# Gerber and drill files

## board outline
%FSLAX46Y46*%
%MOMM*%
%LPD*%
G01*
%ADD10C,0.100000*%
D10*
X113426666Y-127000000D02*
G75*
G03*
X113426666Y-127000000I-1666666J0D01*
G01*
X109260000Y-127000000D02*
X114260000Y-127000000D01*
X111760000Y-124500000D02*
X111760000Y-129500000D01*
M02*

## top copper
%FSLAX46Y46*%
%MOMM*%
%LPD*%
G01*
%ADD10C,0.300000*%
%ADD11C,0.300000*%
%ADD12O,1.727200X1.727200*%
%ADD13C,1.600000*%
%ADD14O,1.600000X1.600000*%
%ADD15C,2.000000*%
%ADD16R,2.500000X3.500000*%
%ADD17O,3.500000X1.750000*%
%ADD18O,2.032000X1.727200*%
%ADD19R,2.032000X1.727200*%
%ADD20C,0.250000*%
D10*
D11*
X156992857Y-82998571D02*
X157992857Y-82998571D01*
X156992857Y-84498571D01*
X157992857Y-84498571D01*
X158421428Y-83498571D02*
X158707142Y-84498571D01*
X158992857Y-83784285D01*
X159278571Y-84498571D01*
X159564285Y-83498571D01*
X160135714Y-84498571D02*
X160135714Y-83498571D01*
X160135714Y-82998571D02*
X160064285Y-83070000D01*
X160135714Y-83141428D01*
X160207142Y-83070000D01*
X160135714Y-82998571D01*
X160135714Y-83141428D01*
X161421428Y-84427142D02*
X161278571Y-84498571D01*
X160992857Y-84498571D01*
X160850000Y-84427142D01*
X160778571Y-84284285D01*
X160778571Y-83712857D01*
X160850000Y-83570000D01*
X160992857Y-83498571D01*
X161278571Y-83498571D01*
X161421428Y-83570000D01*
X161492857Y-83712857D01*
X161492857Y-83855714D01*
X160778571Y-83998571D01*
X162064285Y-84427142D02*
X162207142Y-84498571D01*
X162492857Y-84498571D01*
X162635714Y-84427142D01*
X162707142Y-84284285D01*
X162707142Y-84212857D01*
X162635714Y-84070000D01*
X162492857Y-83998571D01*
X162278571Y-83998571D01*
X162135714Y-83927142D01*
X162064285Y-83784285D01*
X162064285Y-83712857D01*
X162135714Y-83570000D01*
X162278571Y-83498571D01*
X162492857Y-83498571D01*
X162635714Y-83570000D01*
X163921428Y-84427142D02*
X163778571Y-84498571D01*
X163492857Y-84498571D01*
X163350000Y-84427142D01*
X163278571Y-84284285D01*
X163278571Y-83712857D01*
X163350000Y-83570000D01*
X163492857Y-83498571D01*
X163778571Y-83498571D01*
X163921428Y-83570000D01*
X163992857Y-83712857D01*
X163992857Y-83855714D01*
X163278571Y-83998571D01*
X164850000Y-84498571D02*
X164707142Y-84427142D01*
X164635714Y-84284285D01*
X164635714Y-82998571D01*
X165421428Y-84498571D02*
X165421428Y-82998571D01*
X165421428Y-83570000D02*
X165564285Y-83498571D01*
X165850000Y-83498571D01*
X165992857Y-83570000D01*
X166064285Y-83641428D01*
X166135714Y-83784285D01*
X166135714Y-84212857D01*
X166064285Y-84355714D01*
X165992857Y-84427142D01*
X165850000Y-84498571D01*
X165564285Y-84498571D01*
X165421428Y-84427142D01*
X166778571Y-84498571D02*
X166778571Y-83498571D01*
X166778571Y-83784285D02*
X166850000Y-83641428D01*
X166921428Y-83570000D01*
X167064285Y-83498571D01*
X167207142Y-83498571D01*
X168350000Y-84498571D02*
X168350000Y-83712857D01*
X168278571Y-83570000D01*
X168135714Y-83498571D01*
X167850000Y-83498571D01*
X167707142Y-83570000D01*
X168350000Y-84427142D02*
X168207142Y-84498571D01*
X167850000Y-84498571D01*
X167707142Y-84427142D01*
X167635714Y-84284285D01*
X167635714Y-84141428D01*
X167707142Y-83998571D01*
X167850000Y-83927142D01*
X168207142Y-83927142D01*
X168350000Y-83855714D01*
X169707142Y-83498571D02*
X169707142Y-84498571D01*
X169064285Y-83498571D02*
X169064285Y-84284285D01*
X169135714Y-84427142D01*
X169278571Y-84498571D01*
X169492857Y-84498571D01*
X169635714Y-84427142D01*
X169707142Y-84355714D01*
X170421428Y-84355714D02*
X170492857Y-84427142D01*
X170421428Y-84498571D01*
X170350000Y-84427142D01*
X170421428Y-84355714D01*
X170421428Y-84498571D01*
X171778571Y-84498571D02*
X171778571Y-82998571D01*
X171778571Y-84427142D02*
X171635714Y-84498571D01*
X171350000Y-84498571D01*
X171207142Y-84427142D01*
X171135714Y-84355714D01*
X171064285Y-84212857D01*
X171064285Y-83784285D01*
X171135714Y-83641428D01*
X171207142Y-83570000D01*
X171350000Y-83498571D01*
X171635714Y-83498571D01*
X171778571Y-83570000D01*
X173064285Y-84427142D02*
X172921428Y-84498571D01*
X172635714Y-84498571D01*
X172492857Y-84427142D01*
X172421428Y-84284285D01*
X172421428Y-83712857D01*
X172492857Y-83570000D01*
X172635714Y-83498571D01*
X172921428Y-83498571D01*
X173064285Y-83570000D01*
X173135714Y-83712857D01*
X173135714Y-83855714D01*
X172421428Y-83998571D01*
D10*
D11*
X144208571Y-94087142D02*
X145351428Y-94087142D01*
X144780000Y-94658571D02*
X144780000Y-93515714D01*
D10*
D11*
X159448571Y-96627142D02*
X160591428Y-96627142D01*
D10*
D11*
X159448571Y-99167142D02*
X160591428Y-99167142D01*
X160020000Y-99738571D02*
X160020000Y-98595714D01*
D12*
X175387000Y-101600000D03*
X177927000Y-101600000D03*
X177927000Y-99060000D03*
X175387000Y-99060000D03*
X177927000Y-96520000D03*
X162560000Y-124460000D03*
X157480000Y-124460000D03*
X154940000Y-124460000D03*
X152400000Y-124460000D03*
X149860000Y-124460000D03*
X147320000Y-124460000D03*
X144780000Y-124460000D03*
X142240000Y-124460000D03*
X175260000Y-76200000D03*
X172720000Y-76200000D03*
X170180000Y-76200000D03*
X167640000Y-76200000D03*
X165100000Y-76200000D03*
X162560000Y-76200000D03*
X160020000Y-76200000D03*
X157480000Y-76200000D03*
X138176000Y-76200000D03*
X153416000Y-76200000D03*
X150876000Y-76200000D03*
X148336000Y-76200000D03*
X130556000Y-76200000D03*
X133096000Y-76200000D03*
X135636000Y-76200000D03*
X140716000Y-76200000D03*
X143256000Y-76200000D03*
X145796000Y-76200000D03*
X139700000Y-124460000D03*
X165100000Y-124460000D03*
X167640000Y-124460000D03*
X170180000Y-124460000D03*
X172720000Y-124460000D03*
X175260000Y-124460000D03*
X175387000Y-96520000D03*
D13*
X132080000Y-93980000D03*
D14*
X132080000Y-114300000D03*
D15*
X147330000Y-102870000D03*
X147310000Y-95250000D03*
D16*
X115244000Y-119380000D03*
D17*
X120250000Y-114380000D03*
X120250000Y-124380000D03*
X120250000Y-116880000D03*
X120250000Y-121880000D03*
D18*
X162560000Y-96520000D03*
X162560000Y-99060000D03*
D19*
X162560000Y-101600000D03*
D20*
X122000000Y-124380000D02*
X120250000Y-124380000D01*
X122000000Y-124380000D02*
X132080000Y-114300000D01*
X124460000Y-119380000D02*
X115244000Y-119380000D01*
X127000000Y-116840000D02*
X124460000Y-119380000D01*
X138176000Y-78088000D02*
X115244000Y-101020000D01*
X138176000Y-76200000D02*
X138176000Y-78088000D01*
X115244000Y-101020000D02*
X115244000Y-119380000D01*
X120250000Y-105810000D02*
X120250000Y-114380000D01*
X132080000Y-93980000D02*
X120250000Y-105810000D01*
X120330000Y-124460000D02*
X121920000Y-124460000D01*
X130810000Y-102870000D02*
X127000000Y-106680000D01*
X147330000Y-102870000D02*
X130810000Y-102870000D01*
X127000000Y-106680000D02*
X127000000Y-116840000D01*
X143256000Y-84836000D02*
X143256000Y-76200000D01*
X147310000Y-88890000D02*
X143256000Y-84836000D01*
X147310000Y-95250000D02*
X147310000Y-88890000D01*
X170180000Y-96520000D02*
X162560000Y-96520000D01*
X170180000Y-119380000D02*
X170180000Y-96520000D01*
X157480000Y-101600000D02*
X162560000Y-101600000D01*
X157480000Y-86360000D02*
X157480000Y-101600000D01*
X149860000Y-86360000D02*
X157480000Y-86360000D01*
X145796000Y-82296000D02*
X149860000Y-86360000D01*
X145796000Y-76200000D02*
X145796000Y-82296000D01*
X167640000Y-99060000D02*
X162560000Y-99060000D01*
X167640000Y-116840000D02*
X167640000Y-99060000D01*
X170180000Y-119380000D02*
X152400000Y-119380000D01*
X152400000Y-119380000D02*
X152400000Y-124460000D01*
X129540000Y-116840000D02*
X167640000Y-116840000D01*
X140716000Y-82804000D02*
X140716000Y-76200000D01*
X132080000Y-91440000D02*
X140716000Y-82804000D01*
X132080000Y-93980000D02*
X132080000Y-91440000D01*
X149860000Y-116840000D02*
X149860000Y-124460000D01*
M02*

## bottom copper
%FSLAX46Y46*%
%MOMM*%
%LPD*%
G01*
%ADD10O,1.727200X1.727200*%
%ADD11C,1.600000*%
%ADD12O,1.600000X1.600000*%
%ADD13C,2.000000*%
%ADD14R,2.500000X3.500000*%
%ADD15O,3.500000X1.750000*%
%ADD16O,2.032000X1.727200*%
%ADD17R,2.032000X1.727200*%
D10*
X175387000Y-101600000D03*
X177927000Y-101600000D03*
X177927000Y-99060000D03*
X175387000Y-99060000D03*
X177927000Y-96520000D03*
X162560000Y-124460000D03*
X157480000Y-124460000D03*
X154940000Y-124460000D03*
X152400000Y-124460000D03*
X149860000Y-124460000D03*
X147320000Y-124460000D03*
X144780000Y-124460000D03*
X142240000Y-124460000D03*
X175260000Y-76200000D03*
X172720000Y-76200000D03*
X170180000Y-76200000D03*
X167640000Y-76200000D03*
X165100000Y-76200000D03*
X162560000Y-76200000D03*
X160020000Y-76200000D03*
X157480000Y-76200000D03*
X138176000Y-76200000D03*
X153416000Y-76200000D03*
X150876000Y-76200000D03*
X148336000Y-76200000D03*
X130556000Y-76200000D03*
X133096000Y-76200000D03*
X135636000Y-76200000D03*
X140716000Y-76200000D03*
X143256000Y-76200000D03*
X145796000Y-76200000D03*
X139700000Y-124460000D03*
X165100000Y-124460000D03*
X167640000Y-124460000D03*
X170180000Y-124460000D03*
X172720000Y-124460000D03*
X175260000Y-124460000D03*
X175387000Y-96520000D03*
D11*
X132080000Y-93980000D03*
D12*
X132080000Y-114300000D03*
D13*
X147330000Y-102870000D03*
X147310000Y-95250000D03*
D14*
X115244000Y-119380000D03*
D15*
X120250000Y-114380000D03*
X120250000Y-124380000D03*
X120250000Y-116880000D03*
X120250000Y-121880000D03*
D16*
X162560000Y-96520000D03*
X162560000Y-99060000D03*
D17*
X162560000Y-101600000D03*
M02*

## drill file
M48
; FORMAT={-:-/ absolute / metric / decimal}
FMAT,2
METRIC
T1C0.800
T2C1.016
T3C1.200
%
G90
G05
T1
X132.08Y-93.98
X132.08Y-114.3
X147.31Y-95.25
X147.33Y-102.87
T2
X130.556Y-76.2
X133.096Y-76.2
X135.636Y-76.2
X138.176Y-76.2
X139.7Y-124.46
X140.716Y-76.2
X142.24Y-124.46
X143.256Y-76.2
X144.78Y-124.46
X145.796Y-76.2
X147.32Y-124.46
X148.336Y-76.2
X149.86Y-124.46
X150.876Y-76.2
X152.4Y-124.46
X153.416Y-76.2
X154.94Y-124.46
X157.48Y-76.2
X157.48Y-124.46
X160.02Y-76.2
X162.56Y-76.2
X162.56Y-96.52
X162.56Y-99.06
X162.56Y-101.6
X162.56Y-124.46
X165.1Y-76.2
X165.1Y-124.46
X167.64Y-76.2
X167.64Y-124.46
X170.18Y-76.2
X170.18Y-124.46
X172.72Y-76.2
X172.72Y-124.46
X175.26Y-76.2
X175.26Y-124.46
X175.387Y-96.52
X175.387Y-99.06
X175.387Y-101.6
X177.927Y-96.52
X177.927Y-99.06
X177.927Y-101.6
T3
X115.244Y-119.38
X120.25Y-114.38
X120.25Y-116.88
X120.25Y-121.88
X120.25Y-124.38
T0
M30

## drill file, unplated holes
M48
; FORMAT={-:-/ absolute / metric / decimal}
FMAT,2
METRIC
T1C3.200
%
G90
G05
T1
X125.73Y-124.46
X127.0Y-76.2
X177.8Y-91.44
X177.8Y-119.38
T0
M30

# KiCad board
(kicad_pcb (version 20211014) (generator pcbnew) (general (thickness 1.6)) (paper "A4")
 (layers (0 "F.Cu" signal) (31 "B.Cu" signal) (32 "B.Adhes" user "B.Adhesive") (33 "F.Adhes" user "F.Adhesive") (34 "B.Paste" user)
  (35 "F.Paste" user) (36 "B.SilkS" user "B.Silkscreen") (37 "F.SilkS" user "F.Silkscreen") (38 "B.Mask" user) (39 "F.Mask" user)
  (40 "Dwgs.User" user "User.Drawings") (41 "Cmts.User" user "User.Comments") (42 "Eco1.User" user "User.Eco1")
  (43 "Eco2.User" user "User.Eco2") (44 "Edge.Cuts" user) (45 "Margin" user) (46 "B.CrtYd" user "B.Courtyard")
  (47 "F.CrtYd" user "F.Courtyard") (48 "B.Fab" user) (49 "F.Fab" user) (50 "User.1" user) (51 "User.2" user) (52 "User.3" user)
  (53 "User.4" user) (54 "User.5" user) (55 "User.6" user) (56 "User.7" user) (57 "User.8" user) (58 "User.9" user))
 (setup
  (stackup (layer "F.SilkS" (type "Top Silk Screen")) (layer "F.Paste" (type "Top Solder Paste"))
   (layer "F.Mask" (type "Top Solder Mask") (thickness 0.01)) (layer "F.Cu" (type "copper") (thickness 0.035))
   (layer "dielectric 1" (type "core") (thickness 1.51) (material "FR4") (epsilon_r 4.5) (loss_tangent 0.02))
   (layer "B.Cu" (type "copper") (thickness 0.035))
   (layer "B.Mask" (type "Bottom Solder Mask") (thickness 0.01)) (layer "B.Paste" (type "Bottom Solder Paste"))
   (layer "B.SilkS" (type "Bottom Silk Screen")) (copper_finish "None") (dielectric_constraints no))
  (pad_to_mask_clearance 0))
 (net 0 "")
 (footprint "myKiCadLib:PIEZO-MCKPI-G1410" (layer "F.Cu") (at 147.32 99.06 90)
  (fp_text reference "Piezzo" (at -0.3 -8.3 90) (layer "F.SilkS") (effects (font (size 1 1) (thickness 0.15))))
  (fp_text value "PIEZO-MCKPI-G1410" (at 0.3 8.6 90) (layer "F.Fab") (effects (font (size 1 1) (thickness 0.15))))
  (pad "1" thru_hole circle locked (at -3.81 0.01 90) (size 2 2) (drill 0.8) (layers *.Cu *.Mask "F.SilkS"))
  (pad "2" thru_hole circle locked (at 3.81 -0.01 90) (size 2 2) (drill 0.8) (layers *.Cu *.Mask "F.SilkS")))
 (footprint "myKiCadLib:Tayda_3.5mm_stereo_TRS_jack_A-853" (layer "F.Cu") (at 116.84 119.38 90)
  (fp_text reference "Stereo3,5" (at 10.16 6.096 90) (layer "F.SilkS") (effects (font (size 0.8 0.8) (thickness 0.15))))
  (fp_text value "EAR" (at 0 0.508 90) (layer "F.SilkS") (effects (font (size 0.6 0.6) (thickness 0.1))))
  (pad "1" thru_hole rect locked (at 0 -1.596 90) (size 3.5 2.5) (drill 1.2) (layers *.Cu *.Mask "F.SilkS"))
  (pad "2" thru_hole oval locked (at 5 3.41 90) (size 1.75 3.5) (drill 1.2) (layers *.Cu *.Mask "F.SilkS"))
  (pad "3" thru_hole oval locked (at 2.5 3.41 90) (size 1.75 3.5) (drill 1.2) (layers *.Cu *.Mask "F.SilkS"))
  (pad "4" thru_hole oval locked (at -2.5 3.41 90) (size 1.75 3.5) (drill 1.2) (layers *.Cu *.Mask "F.SilkS"))
  (pad "5" thru_hole oval locked (at -5 3.41 90) (size 1.75 3.5) (drill 1.2) (layers *.Cu *.Mask "F.SilkS")))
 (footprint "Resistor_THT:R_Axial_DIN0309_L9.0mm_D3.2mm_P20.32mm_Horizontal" (layer "F.Cu") (at 132.08 93.98 -90)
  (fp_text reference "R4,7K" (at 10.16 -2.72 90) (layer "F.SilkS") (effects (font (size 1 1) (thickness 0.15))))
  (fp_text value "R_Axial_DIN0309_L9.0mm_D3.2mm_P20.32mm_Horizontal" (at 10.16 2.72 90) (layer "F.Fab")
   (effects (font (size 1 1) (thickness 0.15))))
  (pad "1" thru_hole circle (at 0 0 270) (size 1.6 1.6) (drill 0.8) (layers *.Cu *.Mask))
  (pad "2" thru_hole oval (at 20.32 0 270) (size 1.6 1.6) (drill 0.8) (layers *.Cu *.Mask)))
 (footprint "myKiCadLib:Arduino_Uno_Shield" (layer "F.Cu") (at 111.76 127)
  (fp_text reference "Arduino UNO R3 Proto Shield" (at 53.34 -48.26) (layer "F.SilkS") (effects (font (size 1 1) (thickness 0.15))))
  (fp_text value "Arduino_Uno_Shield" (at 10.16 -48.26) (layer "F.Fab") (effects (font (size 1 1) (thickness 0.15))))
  (pad "" np_thru_hole circle locked (at 15.24 -50.8) (size 3.2 3.2) (drill 3.2) (layers *.Cu *.Mask))
  (pad "" np_thru_hole circle locked (at 66.04 -7.62) (size 3.2 3.2) (drill 3.2) (layers *.Cu *.Mask))
  (pad "" np_thru_hole circle locked (at 13.97 -2.54) (size 3.2 3.2) (drill 3.2) (layers *.Cu *.Mask))
  (pad "" thru_hole oval locked (at 27.94 -2.54) (size 1.7272 1.7272) (drill 1.016) (layers *.Cu *.Mask))
  (pad "" np_thru_hole circle locked (at 66.04 -35.56) (size 3.2 3.2) (drill 3.2) (layers *.Cu *.Mask))
  (pad "3V3" thru_hole oval locked (at 35.56 -2.54) (size 1.7272 1.7272) (drill 1.016) (layers *.Cu *.Mask))
  (pad "5V1" thru_hole oval locked (at 38.1 -2.54) (size 1.7272 1.7272) (drill 1.016) (layers *.Cu *.Mask))
  (pad "5V2" thru_hole oval locked (at 66.167 -30.48) (size 1.7272 1.7272) (drill 1.016) (layers *.Cu *.Mask))
  (pad "A0" thru_hole oval locked (at 50.8 -2.54) (size 1.7272 1.7272) (drill 1.016) (layers *.Cu *.Mask))
  (pad "A1" thru_hole oval locked (at 53.34 -2.54) (size 1.7272 1.7272) (drill 1.016) (layers *.Cu *.Mask))
  (pad "A2" thru_hole oval locked (at 55.88 -2.54) (size 1.7272 1.7272) (drill 1.016) (layers *.Cu *.Mask))
  (pad "A3" thru_hole oval locked (at 58.42 -2.54) (size 1.7272 1.7272) (drill 1.016) (layers *.Cu *.Mask))
  (pad "A4" thru_hole oval locked (at 60.96 -2.54) (size 1.7272 1.7272) (drill 1.016) (layers *.Cu *.Mask))
  (pad "A5" thru_hole oval locked (at 63.5 -2.54) (size 1.7272 1.7272) (drill 1.016) (layers *.Cu *.Mask))
  (pad "AREF" thru_hole oval locked (at 23.876 -50.8) (size 1.7272 1.7272) (drill 1.016) (layers *.Cu *.Mask))
  (pad "D0" thru_hole oval locked (at 63.5 -50.8) (size 1.7272 1.7272) (drill 1.016) (layers *.Cu *.Mask))
  (pad "D1" thru_hole oval locked (at 60.96 -50.8) (size 1.7272 1.7272) (drill 1.016) (layers *.Cu *.Mask))
  (pad "D2" thru_hole oval locked (at 58.42 -50.8) (size 1.7272 1.7272) (drill 1.016) (layers *.Cu *.Mask))
  (pad "D3" thru_hole oval locked (at 55.88 -50.8) (size 1.7272 1.7272) (drill 1.016) (layers *.Cu *.Mask))
  (pad "D4" thru_hole oval locked (at 53.34 -50.8) (size 1.7272 1.7272) (drill 1.016) (layers *.Cu *.Mask))
  (pad "D5" thru_hole oval locked (at 50.8 -50.8) (size 1.7272 1.7272) (drill 1.016) (layers *.Cu *.Mask))
  (pad "D6" thru_hole oval locked (at 48.26 -50.8) (size 1.7272 1.7272) (drill 1.016) (layers *.Cu *.Mask))
  (pad "D7" thru_hole oval locked (at 45.72 -50.8) (size 1.7272 1.7272) (drill 1.016) (layers *.Cu *.Mask))
  (pad "D8" thru_hole oval locked (at 41.656 -50.8) (size 1.7272 1.7272) (drill 1.016) (layers *.Cu *.Mask))
  (pad "D9" thru_hole oval locked (at 39.116 -50.8) (size 1.7272 1.7272) (drill 1.016) (layers *.Cu *.Mask))
  (pad "D10" thru_hole oval locked (at 36.576 -50.8) (size 1.7272 1.7272) (drill 1.016) (layers *.Cu *.Mask))
  (pad "D11" thru_hole oval locked (at 34.036 -50.8) (size 1.7272 1.7272) (drill 1.016) (layers *.Cu *.Mask))
  (pad "D12" thru_hole oval locked (at 31.496 -50.8) (size 1.7272 1.7272) (drill 1.016) (layers *.Cu *.Mask))
  (pad "D13" thru_hole oval locked (at 28.956 -50.8) (size 1.7272 1.7272) (drill 1.016) (layers *.Cu *.Mask))
  (pad "GND1" thru_hole oval locked (at 26.416 -50.8) (size 1.7272 1.7272) (drill 1.016) (layers *.Cu *.Mask))
  (pad "GND2" thru_hole oval locked (at 40.64 -2.54) (size 1.7272 1.7272) (drill 1.016) (layers *.Cu *.Mask))
  (pad "GND3" thru_hole oval locked (at 43.18 -2.54) (size 1.7272 1.7272) (drill 1.016) (layers *.Cu *.Mask))
  (pad "GND4" thru_hole oval locked (at 66.167 -25.4) (size 1.7272 1.7272) (drill 1.016) (layers *.Cu *.Mask))
  (pad "IORF" thru_hole oval locked (at 30.48 -2.54) (size 1.7272 1.7272) (drill 1.016) (layers *.Cu *.Mask))
  (pad "MISO" thru_hole oval locked (at 63.627 -30.48) (size 1.7272 1.7272) (drill 1.016) (layers *.Cu *.Mask))
  (pad "MOSI" thru_hole oval locked (at 66.167 -27.94) (size 1.7272 1.7272) (drill 1.016) (layers *.Cu *.Mask))
  (pad "RST1" thru_hole oval locked (at 33.02 -2.54) (size 1.7272 1.7272) (drill 1.016) (layers *.Cu *.Mask))
  (pad "RST2" thru_hole oval locked (at 63.627 -25.4) (size 1.7272 1.7272) (drill 1.016) (layers *.Cu *.Mask))
  (pad "SCK" thru_hole oval locked (at 63.627 -27.94) (size 1.7272 1.7272) (drill 1.016) (layers *.Cu *.Mask))
  (pad "SCL" thru_hole oval locked (at 18.796 -50.8) (size 1.7272 1.7272) (drill 1.016) (layers *.Cu *.Mask))
  (pad "SDA" thru_hole oval locked (at 21.336 -50.8) (size 1.7272 1.7272) (drill 1.016) (layers *.Cu *.Mask))
  (pad "VIN" thru_hole oval locked (at 45.72 -2.54) (size 1.7272 1.7272) (drill 1.016) (layers *.Cu *.Mask)))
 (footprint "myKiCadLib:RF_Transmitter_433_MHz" (layer "F.Cu") (at 162.56 99.06 90)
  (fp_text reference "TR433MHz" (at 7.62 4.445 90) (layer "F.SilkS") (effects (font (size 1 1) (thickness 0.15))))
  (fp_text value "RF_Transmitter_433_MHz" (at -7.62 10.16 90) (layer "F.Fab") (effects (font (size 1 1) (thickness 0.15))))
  (pad "1" thru_hole rect locked (at -2.54 0 180) (size 2.032 1.7272) (drill 1.016) (layers *.Cu *.Mask "F.SilkS"))
  (pad "2" thru_hole oval locked (at 0 0 180) (size 2.032 1.7272) (drill 1.016) (layers *.Cu *.Mask "F.SilkS"))
  (pad "3" thru_hole oval locked (at 2.54 0 180) (size 2.032 1.7272) (drill 1.016) (layers *.Cu *.Mask "F.SilkS")))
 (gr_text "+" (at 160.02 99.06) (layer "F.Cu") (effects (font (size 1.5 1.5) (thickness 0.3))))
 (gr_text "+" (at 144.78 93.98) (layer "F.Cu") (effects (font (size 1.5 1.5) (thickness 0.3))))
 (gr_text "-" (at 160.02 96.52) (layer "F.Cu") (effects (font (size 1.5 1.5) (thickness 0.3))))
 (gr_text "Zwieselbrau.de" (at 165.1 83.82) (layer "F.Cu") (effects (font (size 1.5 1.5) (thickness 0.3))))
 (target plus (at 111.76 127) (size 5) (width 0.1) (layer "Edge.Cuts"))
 (segment (start 127 106.68) (end 127 116.84) (width 0.25) (layer "F.Cu") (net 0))
 (segment (start 138.176 78.088) (end 115.244 101.02) (width 0.25) (layer "F.Cu") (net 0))
 (segment (start 127 116.84) (end 124.46 119.38) (width 0.25) (layer "F.Cu") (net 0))
 (segment (start 132.08 93.98) (end 132.08 91.44) (width 0.25) (layer "F.Cu") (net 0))
 (segment (start 122 124.38) (end 120.25 124.38) (width 0.25) (layer "F.Cu") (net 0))
 (segment (start 149.86 116.84) (end 149.86 124.46) (width 0.25) (layer "F.Cu") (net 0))
 (segment (start 129.54 116.84) (end 167.64 116.84) (width 0.25) (layer "F.Cu") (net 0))
 (segment (start 122 124.38) (end 132.08 114.3) (width 0.25) (layer "F.Cu") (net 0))
 (segment (start 157.48 86.36) (end 157.48 101.6) (width 0.25) (layer "F.Cu") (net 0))
 (segment (start 132.08 93.98) (end 120.25 105.81) (width 0.25) (layer "F.Cu") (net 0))
 (segment (start 170.18 119.38) (end 152.4 119.38) (width 0.25) (layer "F.Cu") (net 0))
 (segment (start 167.64 116.84) (end 167.64 99.06) (width 0.25) (layer "F.Cu") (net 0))
 (segment (start 170.18 119.38) (end 170.18 96.52) (width 0.25) (layer "F.Cu") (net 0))
 (segment (start 130.81 102.87) (end 127 106.68) (width 0.25) (layer "F.Cu") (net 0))
 (segment (start 145.796 76.2) (end 145.796 82.296) (width 0.25) (layer "F.Cu") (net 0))
 (segment (start 147.33 102.87) (end 130.81 102.87) (width 0.25) (layer "F.Cu") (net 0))
 (segment (start 115.244 101.02) (end 115.244 119.38) (width 0.25) (layer "F.Cu") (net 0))
 (segment (start 140.716 82.804) (end 140.716 76.2) (width 0.25) (layer "F.Cu") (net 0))
 (segment (start 132.08 91.44) (end 140.716 82.804) (width 0.25) (layer "F.Cu") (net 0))
 (segment (start 149.86 86.36) (end 157.48 86.36) (width 0.25) (layer "F.Cu") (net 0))
 (segment (start 170.18 96.52) (end 162.56 96.52) (width 0.25) (layer "F.Cu") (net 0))
 (segment (start 147.31 95.25) (end 147.31 88.89) (width 0.25) (layer "F.Cu") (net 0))
 (segment (start 138.176 76.2) (end 138.176 78.088) (width 0.25) (layer "F.Cu") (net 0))
 (segment (start 145.796 82.296) (end 149.86 86.36) (width 0.25) (layer "F.Cu") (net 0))
 (segment (start 120.33 124.46) (end 121.92 124.46) (width 0.25) (layer "F.Cu") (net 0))
 (segment (start 152.4 119.38) (end 152.4 124.46) (width 0.25) (layer "F.Cu") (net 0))
 (segment (start 167.64 99.06) (end 162.56 99.06) (width 0.25) (layer "F.Cu") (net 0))
 (segment (start 120.25 105.81) (end 120.25 114.38) (width 0.25) (layer "F.Cu") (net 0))
 (segment (start 147.31 88.89) (end 143.256 84.836) (width 0.25) (layer "F.Cu") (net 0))
 (segment (start 143.256 84.836) (end 143.256 76.2) (width 0.25) (layer "F.Cu") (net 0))
 (segment (start 157.48 101.6) (end 162.56 101.6) (width 0.25) (layer "F.Cu") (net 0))
 (segment (start 124.46 119.38) (end 115.244 119.38) (width 0.25) (layer "F.Cu") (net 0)))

